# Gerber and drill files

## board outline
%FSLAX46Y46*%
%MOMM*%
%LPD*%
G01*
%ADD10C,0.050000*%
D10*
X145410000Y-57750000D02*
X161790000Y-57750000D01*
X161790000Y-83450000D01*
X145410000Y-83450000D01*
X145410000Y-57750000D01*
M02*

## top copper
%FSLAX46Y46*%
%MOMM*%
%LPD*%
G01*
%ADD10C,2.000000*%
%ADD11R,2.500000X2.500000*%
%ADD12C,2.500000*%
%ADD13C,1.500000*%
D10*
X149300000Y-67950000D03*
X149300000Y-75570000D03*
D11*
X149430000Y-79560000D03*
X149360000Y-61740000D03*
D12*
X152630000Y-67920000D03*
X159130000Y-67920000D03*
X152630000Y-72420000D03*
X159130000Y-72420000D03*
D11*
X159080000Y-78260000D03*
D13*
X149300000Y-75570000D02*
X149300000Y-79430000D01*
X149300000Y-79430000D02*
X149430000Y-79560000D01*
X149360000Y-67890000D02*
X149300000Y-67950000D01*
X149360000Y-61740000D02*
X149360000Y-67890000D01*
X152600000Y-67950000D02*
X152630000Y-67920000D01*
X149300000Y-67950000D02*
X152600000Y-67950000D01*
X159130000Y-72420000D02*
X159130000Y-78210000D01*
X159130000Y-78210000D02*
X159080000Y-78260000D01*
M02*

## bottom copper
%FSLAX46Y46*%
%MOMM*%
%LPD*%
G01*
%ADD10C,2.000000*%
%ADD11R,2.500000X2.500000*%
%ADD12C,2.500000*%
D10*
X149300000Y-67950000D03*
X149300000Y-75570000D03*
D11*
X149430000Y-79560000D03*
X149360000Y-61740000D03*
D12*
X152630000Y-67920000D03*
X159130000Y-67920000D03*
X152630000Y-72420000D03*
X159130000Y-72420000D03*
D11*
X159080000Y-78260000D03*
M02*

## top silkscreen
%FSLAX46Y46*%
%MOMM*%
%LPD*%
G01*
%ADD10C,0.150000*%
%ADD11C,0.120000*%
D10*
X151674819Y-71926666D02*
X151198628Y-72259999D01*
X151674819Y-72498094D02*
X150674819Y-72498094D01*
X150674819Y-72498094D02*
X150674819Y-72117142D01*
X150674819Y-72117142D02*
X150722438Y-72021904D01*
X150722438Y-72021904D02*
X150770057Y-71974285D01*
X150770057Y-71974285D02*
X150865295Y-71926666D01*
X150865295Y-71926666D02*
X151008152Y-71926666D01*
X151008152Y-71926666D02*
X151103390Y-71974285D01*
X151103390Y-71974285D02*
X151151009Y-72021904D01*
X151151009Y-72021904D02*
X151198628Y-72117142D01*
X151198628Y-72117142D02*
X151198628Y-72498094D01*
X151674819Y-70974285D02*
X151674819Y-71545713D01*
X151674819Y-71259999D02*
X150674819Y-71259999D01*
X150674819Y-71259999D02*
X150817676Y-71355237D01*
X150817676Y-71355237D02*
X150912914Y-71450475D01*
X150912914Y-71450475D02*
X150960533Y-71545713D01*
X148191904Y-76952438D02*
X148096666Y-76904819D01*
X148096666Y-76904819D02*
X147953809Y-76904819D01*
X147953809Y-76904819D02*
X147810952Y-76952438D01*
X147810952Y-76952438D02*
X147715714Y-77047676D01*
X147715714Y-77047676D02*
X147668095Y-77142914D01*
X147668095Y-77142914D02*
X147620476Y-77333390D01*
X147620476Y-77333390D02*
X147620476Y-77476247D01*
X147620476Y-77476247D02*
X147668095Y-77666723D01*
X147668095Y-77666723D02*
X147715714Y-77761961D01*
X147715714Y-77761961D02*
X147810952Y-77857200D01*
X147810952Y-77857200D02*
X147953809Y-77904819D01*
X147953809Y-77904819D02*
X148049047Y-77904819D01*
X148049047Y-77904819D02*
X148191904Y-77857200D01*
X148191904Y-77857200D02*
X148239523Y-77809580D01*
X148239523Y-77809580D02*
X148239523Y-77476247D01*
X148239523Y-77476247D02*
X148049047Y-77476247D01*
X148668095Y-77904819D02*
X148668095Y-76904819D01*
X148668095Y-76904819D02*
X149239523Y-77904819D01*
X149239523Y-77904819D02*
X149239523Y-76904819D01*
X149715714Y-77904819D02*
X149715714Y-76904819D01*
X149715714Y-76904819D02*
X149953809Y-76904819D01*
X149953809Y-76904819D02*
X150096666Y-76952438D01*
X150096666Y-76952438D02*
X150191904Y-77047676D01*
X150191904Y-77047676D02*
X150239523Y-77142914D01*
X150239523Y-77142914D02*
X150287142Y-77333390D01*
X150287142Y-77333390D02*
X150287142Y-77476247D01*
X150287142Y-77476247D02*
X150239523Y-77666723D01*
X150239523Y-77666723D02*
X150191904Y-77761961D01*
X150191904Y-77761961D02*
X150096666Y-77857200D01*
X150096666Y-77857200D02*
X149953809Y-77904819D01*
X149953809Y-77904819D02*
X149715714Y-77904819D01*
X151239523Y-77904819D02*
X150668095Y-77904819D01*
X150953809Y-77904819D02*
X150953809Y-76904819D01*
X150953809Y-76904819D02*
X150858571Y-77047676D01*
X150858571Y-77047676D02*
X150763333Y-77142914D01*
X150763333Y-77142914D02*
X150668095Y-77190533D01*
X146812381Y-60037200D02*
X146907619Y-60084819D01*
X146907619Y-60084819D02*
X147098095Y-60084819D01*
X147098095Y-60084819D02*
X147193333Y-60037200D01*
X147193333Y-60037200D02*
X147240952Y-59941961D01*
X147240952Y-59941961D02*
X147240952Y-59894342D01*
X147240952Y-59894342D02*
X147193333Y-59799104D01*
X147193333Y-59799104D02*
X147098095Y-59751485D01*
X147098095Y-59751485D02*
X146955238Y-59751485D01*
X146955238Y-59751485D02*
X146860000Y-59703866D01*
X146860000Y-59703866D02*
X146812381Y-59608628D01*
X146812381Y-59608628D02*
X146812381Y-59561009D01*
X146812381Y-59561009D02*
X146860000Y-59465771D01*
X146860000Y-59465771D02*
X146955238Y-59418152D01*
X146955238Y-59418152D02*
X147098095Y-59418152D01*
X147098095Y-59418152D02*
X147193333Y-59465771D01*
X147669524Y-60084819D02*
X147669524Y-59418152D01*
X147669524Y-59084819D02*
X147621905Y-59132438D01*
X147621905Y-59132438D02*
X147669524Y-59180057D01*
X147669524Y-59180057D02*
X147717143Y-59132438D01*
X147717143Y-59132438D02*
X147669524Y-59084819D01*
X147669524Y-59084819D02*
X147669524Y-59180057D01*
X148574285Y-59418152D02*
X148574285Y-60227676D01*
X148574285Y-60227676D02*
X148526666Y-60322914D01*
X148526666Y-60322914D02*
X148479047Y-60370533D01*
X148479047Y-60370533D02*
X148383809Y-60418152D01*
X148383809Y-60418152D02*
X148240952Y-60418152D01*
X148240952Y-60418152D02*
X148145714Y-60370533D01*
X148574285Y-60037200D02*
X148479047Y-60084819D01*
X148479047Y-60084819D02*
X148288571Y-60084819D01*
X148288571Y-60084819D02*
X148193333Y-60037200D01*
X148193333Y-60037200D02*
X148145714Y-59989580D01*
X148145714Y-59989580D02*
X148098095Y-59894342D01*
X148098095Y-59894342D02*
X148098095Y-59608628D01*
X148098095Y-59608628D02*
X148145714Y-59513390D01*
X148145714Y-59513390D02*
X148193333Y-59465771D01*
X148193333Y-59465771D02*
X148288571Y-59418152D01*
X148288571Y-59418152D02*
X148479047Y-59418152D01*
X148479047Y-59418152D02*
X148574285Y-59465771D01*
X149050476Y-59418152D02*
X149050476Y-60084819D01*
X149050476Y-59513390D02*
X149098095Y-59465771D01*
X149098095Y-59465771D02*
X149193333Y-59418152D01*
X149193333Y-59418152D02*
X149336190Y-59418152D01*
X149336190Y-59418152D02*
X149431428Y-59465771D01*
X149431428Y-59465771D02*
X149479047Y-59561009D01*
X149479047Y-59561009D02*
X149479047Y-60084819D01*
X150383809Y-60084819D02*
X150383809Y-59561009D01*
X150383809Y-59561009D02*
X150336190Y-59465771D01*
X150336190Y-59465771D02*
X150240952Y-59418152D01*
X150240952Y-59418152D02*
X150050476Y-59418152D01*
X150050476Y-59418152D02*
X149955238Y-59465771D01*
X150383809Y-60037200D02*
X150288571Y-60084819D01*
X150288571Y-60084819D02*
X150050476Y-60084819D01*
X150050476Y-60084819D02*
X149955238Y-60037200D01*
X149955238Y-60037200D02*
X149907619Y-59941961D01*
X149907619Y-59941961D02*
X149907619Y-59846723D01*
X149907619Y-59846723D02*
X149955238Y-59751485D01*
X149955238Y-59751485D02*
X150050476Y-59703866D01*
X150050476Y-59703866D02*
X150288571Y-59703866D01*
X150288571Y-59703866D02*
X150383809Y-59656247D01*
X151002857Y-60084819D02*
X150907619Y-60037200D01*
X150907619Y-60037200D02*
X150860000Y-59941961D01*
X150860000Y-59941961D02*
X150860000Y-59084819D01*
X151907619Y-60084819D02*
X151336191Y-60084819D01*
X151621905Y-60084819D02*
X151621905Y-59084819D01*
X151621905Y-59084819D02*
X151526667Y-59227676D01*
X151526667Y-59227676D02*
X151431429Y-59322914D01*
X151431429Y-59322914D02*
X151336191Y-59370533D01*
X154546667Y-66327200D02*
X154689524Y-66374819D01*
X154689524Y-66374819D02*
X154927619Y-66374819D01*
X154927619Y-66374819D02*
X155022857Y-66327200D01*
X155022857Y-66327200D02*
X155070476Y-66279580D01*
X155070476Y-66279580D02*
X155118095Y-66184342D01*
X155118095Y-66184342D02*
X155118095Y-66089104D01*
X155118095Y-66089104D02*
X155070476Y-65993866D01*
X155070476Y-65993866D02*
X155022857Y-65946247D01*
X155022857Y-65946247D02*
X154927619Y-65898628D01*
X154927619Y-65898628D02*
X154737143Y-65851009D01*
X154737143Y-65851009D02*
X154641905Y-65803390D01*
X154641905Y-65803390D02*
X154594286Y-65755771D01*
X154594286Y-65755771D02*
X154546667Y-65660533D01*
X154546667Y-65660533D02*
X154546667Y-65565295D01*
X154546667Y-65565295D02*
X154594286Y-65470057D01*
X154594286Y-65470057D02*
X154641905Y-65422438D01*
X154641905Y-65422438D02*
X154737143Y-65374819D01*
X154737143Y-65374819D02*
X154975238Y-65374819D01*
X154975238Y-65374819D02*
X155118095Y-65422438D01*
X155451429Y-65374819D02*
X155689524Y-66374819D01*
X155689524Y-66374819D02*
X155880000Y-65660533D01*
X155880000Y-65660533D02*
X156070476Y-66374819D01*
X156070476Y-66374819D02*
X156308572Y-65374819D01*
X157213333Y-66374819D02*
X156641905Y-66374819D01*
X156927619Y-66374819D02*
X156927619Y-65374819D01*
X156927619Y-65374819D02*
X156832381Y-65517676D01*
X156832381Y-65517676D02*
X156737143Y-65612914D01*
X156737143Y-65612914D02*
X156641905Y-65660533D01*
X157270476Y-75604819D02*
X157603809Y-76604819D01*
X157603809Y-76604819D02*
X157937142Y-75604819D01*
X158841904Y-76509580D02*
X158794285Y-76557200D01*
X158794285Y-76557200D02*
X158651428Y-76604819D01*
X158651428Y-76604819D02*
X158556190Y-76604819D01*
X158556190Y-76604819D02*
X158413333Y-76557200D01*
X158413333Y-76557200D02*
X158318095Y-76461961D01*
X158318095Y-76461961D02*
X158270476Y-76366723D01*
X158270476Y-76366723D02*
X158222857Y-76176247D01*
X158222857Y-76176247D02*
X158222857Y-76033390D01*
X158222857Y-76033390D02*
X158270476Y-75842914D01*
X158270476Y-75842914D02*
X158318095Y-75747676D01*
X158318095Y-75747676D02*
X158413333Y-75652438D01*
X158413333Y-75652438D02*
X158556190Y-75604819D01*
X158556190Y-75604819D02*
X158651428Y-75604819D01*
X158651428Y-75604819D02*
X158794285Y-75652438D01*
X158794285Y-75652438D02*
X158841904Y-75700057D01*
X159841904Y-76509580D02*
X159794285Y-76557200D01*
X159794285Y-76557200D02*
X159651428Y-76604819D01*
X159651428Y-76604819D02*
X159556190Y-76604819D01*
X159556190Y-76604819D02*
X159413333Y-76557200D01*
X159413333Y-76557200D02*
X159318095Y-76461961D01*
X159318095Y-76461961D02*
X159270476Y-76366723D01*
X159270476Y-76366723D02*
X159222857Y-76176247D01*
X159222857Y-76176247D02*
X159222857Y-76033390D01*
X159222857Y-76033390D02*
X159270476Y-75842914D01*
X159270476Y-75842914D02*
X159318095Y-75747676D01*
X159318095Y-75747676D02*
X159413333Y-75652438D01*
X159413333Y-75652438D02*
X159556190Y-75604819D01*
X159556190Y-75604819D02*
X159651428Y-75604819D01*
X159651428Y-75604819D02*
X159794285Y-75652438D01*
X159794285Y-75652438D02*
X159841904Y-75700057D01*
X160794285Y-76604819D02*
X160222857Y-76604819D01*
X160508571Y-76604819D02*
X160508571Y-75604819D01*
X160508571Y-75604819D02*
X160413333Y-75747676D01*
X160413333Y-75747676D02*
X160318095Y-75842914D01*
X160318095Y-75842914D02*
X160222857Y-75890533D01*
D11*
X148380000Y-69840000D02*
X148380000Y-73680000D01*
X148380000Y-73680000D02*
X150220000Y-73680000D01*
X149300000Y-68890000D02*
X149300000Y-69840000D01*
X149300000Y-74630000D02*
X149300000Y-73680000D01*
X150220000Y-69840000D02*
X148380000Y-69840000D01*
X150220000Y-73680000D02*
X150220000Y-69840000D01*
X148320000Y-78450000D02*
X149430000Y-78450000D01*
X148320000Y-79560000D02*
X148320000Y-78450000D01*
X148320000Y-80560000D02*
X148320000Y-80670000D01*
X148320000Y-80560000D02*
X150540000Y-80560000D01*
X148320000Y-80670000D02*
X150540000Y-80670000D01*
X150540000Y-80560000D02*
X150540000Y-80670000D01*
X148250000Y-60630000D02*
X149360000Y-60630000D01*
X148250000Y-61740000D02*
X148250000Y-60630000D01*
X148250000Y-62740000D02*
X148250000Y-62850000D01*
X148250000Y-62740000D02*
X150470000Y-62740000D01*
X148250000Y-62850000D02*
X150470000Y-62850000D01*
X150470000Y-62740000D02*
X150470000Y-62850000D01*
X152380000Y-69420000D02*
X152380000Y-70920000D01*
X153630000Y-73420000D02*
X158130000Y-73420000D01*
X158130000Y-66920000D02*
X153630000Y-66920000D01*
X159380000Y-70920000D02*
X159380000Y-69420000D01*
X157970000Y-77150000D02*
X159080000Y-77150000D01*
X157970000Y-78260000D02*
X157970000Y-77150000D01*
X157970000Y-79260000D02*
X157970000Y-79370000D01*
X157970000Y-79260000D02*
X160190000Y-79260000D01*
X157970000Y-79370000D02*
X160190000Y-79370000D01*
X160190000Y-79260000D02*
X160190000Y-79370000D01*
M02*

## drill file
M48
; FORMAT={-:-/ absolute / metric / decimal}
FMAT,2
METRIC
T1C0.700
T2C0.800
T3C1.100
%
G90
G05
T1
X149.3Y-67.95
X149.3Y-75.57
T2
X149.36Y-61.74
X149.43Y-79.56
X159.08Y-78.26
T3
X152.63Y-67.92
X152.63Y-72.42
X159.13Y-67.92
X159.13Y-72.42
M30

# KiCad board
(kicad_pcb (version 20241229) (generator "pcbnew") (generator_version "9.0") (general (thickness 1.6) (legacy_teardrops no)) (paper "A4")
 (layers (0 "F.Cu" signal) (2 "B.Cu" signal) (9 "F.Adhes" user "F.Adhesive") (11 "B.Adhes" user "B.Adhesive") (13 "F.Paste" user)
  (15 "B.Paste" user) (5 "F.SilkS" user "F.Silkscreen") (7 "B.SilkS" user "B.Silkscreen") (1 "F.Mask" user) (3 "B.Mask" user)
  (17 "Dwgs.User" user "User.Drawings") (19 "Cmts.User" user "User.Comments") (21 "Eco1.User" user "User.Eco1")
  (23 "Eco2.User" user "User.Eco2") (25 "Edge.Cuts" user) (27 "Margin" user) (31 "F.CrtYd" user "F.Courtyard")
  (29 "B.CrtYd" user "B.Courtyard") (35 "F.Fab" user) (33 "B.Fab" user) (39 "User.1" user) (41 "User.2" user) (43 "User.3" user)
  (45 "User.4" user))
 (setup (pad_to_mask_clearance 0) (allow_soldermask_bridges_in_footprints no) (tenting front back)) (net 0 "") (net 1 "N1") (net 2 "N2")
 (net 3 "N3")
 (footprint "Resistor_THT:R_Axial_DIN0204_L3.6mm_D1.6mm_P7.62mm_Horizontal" (layer "F.Cu") (at 149.3 67.95 -90)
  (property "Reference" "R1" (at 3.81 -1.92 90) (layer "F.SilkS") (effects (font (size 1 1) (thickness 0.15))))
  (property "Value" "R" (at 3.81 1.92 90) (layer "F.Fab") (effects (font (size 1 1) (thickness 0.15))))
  (fp_line (start 1.89 0.92) (end 5.73 0.92) (stroke (width 0.12) (type solid)) (layer "F.SilkS"))
  (fp_line (start 5.73 0.92) (end 5.73 -0.92) (stroke (width 0.12) (type solid)) (layer "F.SilkS"))
  (fp_line (start 0.94 0) (end 1.89 0) (stroke (width 0.12) (type solid)) (layer "F.SilkS"))
  (fp_line (start 6.68 0) (end 5.73 0) (stroke (width 0.12) (type solid)) (layer "F.SilkS"))
  (fp_line (start 1.89 -0.92) (end 1.89 0.92) (stroke (width 0.12) (type solid)) (layer "F.SilkS"))
  (fp_line (start 5.73 -0.92) (end 1.89 -0.92) (stroke (width 0.12) (type solid)) (layer "F.SilkS"))
  (pad "1" thru_hole circle (at 0 0 270) (size 2 2) (drill 0.7) (layers "*.Cu" "*.Mask") (remove_unused_layers no) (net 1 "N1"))
  (pad "2" thru_hole circle (at 7.62 0 270) (size 2 2) (drill 0.7) (layers "*.Cu" "*.Mask") (remove_unused_layers no) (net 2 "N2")))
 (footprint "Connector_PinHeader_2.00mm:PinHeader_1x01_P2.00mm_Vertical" (layer "F.Cu") (at 149.43 79.56)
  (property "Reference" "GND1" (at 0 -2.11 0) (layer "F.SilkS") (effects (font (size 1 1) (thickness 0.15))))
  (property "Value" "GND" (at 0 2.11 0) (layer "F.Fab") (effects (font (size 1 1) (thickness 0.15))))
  (fp_line (start -1.11 -1.11) (end 0 -1.11) (stroke (width 0.12) (type solid)) (layer "F.SilkS"))
  (fp_line (start -1.11 0) (end -1.11 -1.11) (stroke (width 0.12) (type solid)) (layer "F.SilkS"))
  (fp_line (start -1.11 1) (end -1.11 1.11) (stroke (width 0.12) (type solid)) (layer "F.SilkS"))
  (fp_line (start -1.11 1) (end 1.11 1) (stroke (width 0.12) (type solid)) (layer "F.SilkS"))
  (fp_line (start -1.11 1.11) (end 1.11 1.11) (stroke (width 0.12) (type solid)) (layer "F.SilkS"))
  (fp_line (start 1.11 1) (end 1.11 1.11) (stroke (width 0.12) (type solid)) (layer "F.SilkS"))
  (pad "1" thru_hole rect (at 0 0) (size 2.5 2.5) (drill 0.8) (layers "*.Cu" "*.Mask") (remove_unused_layers no) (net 2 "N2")))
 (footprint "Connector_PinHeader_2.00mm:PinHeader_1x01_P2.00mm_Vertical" (layer "F.Cu") (at 149.36 61.74)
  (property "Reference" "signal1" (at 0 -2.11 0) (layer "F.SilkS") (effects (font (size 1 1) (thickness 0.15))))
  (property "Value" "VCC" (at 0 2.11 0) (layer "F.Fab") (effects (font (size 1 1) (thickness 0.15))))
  (fp_line (start -1.11 -1.11) (end 0 -1.11) (stroke (width 0.12) (type solid)) (layer "F.SilkS"))
  (fp_line (start -1.11 0) (end -1.11 -1.11) (stroke (width 0.12) (type solid)) (layer "F.SilkS"))
  (fp_line (start -1.11 1) (end -1.11 1.11) (stroke (width 0.12) (type solid)) (layer "F.SilkS"))
  (fp_line (start -1.11 1) (end 1.11 1) (stroke (width 0.12) (type solid)) (layer "F.SilkS"))
  (fp_line (start -1.11 1.11) (end 1.11 1.11) (stroke (width 0.12) (type solid)) (layer "F.SilkS"))
  (fp_line (start 1.11 1) (end 1.11 1.11) (stroke (width 0.12) (type solid)) (layer "F.SilkS"))
  (pad "2" thru_hole rect (at 0 0) (size 2.5 2.5) (drill 0.8) (layers "*.Cu" "*.Mask") (remove_unused_layers no) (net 1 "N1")))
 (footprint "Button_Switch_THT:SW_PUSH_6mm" (layer "F.Cu") (at 152.63 67.92)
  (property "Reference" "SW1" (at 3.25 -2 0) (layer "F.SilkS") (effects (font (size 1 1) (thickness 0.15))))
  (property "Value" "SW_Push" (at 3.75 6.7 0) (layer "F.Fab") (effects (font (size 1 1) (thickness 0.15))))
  (fp_line (start -0.25 1.5) (end -0.25 3) (stroke (width 0.12) (type solid)) (layer "F.SilkS"))
  (fp_line (start 1 5.5) (end 5.5 5.5) (stroke (width 0.12) (type solid)) (layer "F.SilkS"))
  (fp_line (start 5.5 -1) (end 1 -1) (stroke (width 0.12) (type solid)) (layer "F.SilkS"))
  (fp_line (start 6.75 3) (end 6.75 1.5) (stroke (width 0.12) (type solid)) (layer "F.SilkS"))
  (pad "1" thru_hole circle (at 0 0 90) (size 2.5 2.5) (drill 1.1) (layers "*.Cu" "*.Mask") (remove_unused_layers no) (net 1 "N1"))
  (pad "1" thru_hole circle (at 6.5 0 90) (size 2.5 2.5) (drill 1.1) (layers "*.Cu" "*.Mask") (remove_unused_layers no) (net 1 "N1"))
  (pad "2" thru_hole circle (at 0 4.5 90) (size 2.5 2.5) (drill 1.1) (layers "*.Cu" "*.Mask") (remove_unused_layers no) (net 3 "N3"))
  (pad "2" thru_hole circle (at 6.5 4.5 90) (size 2.5 2.5) (drill 1.1) (layers "*.Cu" "*.Mask") (remove_unused_layers no) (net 3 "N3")))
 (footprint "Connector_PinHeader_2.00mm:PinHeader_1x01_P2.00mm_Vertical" (layer "F.Cu") (at 159.08 78.26)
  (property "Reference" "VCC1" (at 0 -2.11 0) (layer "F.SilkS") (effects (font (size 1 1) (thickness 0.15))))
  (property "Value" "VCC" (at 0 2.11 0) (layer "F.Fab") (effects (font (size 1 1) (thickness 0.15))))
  (fp_line (start -1.11 -1.11) (end 0 -1.11) (stroke (width 0.12) (type solid)) (layer "F.SilkS"))
  (fp_line (start -1.11 0) (end -1.11 -1.11) (stroke (width 0.12) (type solid)) (layer "F.SilkS"))
  (fp_line (start -1.11 1) (end -1.11 1.11) (stroke (width 0.12) (type solid)) (layer "F.SilkS"))
  (fp_line (start -1.11 1) (end 1.11 1) (stroke (width 0.12) (type solid)) (layer "F.SilkS"))
  (fp_line (start -1.11 1.11) (end 1.11 1.11) (stroke (width 0.12) (type solid)) (layer "F.SilkS"))
  (fp_line (start 1.11 1) (end 1.11 1.11) (stroke (width 0.12) (type solid)) (layer "F.SilkS"))
  (pad "1" thru_hole rect (at 0 0) (size 2.5 2.5) (drill 0.8) (layers "*.Cu" "*.Mask") (remove_unused_layers no) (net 3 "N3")))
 (gr_rect (start 145.41 57.75) (end 161.79 83.45) (stroke (width 0.05) (type default)) (fill no) (layer "Edge.Cuts"))
 (segment (start 149.3 75.57) (end 149.3 79.43) (width 1.5) (layer "F.Cu") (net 2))
 (segment (start 149.3 79.43) (end 149.43 79.56) (width 1.5) (layer "F.Cu") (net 2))
 (segment (start 149.36 67.89) (end 149.3 67.95) (width 1.5) (layer "F.Cu") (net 1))
 (segment (start 149.36 61.74) (end 149.36 67.89) (width 1.5) (layer "F.Cu") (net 1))
 (segment (start 152.6 67.95) (end 152.63 67.92) (width 1.5) (layer "F.Cu") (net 1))
 (segment (start 149.3 67.95) (end 152.6 67.95) (width 1.5) (layer "F.Cu") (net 1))
 (segment (start 159.13 72.42) (end 159.13 78.21) (width 1.5) (layer "F.Cu") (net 3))
 (segment (start 159.13 78.21) (end 159.08 78.26) (width 1.5) (layer "F.Cu") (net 3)))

